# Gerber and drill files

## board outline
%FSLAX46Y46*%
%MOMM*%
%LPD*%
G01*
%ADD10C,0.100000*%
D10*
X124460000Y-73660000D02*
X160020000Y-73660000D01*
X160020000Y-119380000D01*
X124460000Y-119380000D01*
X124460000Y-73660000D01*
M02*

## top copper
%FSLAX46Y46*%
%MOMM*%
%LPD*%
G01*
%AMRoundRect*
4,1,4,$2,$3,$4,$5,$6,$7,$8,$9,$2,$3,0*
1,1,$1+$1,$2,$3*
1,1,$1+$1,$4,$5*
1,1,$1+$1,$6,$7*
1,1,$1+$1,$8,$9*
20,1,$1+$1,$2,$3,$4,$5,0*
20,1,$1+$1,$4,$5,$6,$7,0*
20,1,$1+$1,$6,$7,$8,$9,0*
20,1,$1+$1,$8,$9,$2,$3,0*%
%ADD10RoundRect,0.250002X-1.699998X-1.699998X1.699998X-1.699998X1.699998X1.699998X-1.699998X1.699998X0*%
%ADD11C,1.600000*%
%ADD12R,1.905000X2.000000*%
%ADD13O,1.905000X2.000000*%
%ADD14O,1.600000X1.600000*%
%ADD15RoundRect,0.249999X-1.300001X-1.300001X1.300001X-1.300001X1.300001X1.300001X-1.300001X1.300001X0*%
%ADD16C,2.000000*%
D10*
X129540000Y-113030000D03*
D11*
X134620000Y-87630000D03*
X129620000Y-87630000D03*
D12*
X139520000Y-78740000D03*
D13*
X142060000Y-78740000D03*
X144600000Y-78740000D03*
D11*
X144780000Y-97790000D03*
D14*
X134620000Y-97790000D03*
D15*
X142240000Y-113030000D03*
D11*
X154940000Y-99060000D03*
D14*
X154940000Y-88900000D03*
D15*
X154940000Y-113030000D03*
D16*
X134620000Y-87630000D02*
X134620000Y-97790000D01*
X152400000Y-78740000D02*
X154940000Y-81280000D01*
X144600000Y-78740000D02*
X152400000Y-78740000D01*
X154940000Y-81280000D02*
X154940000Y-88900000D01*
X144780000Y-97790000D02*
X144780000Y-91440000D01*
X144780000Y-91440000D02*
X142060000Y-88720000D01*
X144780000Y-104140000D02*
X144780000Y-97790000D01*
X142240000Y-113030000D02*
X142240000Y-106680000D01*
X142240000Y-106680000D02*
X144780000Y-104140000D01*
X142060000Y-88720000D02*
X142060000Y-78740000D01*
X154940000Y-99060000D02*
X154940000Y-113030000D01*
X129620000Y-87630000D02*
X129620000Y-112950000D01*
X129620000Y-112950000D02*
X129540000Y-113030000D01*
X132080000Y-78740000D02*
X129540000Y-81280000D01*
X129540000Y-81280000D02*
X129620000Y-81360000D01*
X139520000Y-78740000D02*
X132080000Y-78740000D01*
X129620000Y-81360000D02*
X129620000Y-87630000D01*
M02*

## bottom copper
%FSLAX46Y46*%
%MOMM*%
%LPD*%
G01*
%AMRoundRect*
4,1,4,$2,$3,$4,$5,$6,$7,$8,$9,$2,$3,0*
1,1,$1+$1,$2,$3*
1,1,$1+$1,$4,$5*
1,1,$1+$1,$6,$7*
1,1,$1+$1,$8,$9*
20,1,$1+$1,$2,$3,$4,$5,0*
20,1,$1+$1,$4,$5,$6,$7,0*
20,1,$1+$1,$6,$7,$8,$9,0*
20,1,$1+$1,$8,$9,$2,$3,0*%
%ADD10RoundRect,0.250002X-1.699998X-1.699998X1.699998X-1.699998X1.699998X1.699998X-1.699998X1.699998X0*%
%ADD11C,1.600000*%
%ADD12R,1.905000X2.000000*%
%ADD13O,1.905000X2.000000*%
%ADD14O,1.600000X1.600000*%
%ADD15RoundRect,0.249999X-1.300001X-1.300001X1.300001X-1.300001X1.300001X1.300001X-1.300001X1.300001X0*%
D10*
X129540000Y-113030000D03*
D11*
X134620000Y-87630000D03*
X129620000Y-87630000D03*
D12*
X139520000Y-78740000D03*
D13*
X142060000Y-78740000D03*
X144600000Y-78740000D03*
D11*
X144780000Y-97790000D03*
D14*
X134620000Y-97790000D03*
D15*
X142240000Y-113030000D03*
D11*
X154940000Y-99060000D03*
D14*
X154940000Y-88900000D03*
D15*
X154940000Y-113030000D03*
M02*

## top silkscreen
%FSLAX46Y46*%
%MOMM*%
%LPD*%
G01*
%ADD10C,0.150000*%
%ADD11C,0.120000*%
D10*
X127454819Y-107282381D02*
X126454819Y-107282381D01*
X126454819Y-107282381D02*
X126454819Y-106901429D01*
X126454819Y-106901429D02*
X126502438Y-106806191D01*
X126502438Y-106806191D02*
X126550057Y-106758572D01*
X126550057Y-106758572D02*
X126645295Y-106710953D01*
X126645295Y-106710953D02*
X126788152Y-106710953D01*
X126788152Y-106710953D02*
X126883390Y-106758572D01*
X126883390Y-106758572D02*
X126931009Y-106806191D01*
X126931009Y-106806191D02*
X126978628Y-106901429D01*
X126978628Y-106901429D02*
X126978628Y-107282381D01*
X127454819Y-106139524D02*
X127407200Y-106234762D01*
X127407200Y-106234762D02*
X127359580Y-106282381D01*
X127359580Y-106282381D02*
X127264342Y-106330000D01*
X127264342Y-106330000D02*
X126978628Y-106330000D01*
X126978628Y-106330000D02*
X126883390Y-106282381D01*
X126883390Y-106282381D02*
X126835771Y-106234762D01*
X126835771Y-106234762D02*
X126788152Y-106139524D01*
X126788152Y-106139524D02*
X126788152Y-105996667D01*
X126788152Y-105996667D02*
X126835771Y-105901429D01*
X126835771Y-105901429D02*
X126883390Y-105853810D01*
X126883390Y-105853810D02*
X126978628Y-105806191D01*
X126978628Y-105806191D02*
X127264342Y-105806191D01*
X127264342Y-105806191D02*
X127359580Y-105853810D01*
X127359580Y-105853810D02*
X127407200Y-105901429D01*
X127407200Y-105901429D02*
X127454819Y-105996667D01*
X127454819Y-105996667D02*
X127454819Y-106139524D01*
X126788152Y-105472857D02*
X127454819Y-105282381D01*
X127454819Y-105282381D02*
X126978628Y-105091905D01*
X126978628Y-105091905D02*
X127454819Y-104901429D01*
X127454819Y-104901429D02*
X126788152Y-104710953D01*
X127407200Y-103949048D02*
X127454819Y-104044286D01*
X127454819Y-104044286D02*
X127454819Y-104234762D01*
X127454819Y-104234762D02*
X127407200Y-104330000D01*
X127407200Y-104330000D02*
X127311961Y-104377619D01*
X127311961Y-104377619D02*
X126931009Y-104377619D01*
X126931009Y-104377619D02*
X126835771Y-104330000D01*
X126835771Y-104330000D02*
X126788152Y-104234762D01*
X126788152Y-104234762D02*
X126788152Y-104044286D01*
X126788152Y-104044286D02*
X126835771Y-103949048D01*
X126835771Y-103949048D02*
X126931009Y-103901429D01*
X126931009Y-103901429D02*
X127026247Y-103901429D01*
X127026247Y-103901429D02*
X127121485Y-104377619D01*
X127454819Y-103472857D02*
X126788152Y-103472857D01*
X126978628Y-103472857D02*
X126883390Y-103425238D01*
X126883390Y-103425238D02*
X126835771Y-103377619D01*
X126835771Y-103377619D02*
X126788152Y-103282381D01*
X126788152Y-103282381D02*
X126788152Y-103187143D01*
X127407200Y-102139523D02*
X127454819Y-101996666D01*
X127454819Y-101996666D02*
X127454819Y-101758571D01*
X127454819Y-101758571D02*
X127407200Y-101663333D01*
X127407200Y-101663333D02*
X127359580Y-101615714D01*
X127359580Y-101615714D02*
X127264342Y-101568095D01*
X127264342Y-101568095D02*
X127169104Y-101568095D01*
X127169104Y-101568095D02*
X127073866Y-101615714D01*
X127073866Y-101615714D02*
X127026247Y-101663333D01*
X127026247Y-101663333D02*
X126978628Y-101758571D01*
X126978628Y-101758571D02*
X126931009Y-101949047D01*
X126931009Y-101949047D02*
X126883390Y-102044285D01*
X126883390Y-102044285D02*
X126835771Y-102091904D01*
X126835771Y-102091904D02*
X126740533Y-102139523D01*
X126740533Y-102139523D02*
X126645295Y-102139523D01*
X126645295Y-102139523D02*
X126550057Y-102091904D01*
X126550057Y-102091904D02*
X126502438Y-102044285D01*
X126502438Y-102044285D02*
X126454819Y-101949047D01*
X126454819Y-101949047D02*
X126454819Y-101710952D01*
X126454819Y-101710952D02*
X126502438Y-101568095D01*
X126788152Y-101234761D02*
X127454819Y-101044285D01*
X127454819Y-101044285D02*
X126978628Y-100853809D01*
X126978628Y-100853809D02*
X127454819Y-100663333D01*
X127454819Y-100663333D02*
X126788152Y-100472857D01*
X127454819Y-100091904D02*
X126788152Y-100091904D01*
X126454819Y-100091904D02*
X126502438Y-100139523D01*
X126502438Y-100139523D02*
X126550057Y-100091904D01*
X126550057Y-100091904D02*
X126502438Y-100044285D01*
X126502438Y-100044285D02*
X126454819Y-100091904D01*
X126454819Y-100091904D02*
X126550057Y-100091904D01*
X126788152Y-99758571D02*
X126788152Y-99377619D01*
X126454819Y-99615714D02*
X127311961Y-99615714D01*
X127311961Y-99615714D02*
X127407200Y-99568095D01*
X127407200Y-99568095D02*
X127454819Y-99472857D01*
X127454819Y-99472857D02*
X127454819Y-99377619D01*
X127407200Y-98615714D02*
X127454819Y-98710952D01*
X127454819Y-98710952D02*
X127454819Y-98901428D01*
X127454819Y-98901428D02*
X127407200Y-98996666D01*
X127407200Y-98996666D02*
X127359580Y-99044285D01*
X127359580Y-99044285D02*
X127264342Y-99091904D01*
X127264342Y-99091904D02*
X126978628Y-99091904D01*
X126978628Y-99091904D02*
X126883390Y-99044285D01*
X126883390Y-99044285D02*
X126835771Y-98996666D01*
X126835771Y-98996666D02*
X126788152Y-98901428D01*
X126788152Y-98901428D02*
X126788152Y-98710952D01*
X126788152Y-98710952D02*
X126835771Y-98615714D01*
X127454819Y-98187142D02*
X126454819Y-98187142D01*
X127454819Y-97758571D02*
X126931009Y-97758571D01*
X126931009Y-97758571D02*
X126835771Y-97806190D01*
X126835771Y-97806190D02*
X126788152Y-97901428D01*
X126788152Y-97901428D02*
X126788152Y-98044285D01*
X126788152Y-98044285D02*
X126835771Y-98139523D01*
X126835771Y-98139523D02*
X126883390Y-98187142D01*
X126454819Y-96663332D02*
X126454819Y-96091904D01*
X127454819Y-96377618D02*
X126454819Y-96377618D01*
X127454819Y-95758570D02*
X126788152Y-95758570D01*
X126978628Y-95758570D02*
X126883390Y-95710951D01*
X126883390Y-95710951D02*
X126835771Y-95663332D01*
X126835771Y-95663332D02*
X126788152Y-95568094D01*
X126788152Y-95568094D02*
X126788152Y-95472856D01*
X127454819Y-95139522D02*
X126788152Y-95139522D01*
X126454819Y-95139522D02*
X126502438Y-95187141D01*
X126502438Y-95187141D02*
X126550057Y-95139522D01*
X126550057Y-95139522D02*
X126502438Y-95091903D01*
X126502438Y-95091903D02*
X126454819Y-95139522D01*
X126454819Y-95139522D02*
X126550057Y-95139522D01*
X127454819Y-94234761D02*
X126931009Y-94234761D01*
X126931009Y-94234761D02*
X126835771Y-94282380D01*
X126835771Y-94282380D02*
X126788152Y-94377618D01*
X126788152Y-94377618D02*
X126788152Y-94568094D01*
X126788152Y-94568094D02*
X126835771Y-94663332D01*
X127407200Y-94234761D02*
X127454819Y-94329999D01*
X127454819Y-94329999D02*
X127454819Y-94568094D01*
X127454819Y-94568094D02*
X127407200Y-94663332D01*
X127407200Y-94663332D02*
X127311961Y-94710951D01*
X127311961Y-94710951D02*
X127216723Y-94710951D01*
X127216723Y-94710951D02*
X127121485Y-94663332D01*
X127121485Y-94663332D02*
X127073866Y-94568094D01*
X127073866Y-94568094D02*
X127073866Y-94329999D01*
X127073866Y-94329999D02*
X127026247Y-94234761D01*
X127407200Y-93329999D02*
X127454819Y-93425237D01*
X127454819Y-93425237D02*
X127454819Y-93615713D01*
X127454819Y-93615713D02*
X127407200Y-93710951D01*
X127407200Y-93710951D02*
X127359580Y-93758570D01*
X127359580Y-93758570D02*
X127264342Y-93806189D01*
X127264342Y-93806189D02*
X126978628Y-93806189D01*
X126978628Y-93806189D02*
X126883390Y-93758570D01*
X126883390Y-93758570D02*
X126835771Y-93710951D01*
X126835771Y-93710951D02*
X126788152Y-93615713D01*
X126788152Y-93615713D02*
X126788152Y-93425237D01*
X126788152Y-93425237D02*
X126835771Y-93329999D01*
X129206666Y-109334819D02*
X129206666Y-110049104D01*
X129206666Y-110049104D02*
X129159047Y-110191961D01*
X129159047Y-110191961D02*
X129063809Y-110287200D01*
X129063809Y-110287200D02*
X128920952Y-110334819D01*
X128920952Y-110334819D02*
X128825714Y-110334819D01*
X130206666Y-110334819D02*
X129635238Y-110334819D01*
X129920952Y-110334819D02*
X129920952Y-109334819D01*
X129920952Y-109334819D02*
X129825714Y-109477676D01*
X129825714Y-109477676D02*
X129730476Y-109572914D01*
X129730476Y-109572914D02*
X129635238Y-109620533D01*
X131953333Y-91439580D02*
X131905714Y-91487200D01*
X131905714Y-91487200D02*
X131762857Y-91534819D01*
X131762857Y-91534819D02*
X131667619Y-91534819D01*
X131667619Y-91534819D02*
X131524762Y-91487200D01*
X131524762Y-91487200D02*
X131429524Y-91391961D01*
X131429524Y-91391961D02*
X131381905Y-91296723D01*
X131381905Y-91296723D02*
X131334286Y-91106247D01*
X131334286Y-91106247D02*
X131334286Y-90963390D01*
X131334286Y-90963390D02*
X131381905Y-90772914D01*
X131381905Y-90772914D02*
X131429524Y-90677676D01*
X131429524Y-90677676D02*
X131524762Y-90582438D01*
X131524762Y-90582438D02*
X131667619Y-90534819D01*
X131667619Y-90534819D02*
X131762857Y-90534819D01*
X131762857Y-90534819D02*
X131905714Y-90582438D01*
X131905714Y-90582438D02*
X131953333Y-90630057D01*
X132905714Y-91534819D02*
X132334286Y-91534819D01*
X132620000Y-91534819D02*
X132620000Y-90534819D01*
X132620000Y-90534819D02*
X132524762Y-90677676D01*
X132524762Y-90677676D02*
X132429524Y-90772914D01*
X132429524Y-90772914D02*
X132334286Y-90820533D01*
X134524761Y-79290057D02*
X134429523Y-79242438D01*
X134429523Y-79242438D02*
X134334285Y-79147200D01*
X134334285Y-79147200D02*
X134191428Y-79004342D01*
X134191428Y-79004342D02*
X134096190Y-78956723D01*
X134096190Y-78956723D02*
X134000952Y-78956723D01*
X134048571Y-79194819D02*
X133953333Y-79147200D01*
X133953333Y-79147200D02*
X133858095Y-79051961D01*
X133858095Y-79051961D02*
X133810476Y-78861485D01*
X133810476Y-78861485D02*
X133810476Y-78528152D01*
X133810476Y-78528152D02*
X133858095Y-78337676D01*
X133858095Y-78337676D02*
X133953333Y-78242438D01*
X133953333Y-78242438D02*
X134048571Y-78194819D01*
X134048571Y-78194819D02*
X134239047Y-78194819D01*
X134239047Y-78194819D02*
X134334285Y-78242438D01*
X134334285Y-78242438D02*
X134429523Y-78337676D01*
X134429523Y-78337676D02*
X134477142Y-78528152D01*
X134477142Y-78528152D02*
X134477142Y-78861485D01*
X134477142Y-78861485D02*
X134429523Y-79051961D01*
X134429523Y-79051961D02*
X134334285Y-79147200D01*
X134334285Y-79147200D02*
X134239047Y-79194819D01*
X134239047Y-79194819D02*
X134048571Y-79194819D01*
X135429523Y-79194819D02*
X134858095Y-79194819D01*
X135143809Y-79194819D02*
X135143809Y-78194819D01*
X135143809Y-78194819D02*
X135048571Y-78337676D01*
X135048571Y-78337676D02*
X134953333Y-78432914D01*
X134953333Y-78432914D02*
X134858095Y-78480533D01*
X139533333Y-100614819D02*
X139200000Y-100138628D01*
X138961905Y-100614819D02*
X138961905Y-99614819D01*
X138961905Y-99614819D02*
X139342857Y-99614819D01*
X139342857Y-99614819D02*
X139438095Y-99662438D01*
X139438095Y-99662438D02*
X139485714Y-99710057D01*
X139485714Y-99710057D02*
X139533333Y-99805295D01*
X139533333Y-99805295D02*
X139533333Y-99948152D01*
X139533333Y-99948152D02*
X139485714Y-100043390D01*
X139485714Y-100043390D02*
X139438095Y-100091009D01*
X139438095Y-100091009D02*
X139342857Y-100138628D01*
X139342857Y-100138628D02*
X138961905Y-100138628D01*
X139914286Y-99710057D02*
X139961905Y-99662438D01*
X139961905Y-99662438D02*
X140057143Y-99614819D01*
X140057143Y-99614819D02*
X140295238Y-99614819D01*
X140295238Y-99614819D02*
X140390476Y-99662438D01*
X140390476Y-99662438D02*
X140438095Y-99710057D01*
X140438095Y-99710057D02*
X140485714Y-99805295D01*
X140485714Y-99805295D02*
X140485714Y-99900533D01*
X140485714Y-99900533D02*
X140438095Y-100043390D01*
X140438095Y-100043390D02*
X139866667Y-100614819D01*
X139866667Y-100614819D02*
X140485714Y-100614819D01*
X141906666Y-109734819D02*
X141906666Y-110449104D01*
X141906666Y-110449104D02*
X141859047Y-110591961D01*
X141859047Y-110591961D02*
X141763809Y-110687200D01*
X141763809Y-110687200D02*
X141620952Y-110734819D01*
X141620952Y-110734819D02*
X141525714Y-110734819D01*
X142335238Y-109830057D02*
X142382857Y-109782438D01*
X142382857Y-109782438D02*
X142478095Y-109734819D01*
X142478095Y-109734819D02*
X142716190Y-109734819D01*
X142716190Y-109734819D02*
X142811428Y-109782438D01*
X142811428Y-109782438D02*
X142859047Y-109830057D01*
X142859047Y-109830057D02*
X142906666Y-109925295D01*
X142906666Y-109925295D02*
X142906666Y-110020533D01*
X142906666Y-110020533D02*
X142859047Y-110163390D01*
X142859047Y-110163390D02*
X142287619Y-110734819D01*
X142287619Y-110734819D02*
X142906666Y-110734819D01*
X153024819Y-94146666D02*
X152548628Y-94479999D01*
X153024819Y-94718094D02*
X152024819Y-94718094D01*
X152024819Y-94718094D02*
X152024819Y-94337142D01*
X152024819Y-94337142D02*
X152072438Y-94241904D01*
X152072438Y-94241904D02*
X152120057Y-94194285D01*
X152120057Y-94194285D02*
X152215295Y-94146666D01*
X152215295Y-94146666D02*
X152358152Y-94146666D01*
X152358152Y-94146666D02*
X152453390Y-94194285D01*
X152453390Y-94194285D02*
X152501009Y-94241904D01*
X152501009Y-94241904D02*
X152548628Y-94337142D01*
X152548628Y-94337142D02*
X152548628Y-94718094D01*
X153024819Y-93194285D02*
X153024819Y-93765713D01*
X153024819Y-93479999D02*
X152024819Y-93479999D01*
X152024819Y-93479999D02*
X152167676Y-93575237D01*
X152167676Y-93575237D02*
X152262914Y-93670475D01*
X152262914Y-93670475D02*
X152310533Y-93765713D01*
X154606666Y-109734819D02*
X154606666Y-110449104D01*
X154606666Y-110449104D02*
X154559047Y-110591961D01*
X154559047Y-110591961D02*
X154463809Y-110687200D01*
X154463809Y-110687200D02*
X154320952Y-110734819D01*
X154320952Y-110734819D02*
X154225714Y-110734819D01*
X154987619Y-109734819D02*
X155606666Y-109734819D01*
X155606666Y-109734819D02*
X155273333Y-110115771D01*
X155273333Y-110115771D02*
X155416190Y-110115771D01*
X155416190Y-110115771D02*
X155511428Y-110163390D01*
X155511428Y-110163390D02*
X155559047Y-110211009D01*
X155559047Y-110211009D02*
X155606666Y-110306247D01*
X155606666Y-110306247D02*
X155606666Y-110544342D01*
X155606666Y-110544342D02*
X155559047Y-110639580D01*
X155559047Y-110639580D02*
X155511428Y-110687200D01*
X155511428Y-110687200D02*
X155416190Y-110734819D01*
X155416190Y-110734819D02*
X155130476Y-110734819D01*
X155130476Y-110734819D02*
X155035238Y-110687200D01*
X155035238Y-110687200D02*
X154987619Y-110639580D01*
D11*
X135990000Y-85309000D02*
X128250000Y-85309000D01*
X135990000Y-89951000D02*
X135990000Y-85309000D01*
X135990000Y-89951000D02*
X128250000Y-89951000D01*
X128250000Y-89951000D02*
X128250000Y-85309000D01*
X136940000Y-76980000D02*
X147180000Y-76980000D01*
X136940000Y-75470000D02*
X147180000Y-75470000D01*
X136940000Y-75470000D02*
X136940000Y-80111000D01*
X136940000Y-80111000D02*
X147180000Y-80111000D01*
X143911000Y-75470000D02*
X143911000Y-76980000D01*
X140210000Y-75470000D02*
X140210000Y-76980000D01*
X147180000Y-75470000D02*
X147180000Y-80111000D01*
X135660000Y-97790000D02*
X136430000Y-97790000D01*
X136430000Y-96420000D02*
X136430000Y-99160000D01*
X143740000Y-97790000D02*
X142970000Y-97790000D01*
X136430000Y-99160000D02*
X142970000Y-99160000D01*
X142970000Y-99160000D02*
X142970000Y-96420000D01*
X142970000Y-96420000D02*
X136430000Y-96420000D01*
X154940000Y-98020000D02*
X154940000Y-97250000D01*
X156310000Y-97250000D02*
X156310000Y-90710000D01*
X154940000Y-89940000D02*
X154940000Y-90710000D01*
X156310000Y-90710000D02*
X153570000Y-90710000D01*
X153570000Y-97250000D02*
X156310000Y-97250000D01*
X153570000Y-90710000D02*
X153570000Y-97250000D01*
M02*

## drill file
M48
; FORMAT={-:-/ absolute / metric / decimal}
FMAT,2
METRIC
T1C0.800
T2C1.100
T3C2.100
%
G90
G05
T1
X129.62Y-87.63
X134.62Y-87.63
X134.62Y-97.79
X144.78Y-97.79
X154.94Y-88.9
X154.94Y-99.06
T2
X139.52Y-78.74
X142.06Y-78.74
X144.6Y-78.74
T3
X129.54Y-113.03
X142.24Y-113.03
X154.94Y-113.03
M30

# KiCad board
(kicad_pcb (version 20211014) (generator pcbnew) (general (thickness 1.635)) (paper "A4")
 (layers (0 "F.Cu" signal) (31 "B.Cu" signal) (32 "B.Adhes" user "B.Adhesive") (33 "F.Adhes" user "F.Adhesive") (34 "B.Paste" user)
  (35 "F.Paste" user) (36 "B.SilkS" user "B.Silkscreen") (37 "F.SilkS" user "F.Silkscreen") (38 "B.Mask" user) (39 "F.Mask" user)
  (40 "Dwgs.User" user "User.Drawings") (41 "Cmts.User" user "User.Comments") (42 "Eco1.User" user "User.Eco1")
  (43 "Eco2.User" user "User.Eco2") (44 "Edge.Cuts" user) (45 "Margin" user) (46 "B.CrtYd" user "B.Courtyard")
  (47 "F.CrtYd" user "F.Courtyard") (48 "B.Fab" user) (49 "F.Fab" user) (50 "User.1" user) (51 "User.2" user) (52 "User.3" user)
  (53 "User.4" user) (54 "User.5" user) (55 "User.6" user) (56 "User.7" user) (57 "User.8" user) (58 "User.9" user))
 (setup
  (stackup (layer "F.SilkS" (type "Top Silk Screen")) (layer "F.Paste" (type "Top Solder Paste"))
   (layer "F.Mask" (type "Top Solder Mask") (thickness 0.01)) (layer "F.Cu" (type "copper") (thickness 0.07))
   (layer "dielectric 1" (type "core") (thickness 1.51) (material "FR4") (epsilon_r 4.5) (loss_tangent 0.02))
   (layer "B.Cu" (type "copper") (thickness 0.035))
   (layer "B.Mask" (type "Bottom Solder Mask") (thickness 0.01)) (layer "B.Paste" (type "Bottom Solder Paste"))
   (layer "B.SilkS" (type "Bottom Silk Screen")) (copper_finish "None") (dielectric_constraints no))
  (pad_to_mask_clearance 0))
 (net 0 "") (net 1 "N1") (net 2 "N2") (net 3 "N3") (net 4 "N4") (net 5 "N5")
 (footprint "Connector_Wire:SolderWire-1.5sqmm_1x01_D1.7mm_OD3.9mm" (layer "F.Cu") (at 129.54 113.03)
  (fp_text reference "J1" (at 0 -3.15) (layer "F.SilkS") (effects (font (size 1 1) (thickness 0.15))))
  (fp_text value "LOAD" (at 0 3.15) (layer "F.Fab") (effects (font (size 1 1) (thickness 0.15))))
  (pad "1" thru_hole roundrect locked (at 0 0) (size 3.9 3.9) (drill 2.1) (layers *.Cu *.Mask) (roundrect_rratio 0.064103) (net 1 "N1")))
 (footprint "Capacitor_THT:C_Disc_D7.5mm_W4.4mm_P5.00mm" (layer "F.Cu") (at 134.62 87.63 180)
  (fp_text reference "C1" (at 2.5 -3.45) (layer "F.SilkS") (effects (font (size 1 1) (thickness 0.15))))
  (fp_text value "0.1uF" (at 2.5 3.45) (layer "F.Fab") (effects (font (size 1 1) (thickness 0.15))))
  (fp_line (start -1.37 2.321) (end 6.37 2.321) (layer "F.SilkS") (width 0.12))
  (fp_line (start -1.37 -2.321) (end -1.37 2.321) (layer "F.SilkS") (width 0.12))
  (fp_line (start -1.37 -2.321) (end 6.37 -2.321) (layer "F.SilkS") (width 0.12))
  (fp_line (start 6.37 -2.321) (end 6.37 2.321) (layer "F.SilkS") (width 0.12))
  (pad "1" thru_hole circle locked (at 0 0 180) (size 1.6 1.6) (drill 0.8) (layers *.Cu *.Mask) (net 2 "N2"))
  (pad "2" thru_hole circle locked (at 5 0 180) (size 1.6 1.6) (drill 0.8) (layers *.Cu *.Mask) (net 1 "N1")))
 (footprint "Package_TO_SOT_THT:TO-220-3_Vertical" (layer "F.Cu") (at 139.52 78.74)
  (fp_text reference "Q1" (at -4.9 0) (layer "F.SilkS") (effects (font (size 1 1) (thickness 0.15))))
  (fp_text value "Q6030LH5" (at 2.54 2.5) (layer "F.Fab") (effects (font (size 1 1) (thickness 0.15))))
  (fp_line (start -2.58 -1.76) (end 7.66 -1.76) (layer "F.SilkS") (width 0.12))
  (fp_line (start -2.58 -3.27) (end 7.66 -3.27) (layer "F.SilkS") (width 0.12))
  (fp_line (start -2.58 -3.27) (end -2.58 1.371) (layer "F.SilkS") (width 0.12))
  (fp_line (start -2.58 1.371) (end 7.66 1.371) (layer "F.SilkS") (width 0.12))
  (fp_line (start 4.391 -3.27) (end 4.391 -1.76) (layer "F.SilkS") (width 0.12))
  (fp_line (start 0.69 -3.27) (end 0.69 -1.76) (layer "F.SilkS") (width 0.12))
  (fp_line (start 7.66 -3.27) (end 7.66 1.371) (layer "F.SilkS") (width 0.12))
  (pad "1" thru_hole rect locked (at 0 0) (size 1.905 2) (drill 1.1) (layers *.Cu *.Mask) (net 1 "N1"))
  (pad "2" thru_hole oval locked (at 2.54 0) (size 1.905 2) (drill 1.1) (layers *.Cu *.Mask) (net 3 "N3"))
  (pad "3" thru_hole oval locked (at 5.08 0) (size 1.905 2) (drill 1.1) (layers *.Cu *.Mask) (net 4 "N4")))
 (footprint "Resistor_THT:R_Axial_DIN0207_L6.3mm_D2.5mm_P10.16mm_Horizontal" (layer "F.Cu") (at 144.78 97.79 180)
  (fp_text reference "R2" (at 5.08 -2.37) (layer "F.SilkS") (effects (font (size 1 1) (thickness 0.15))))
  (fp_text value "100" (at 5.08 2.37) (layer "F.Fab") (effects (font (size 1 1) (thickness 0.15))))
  (fp_line (start 9.12 0) (end 8.35 0) (layer "F.SilkS") (width 0.12))
  (fp_line (start 8.35 1.37) (end 8.35 -1.37) (layer "F.SilkS") (width 0.12))
  (fp_line (start 1.04 0) (end 1.81 0) (layer "F.SilkS") (width 0.12))
  (fp_line (start 8.35 -1.37) (end 1.81 -1.37) (layer "F.SilkS") (width 0.12))
  (fp_line (start 1.81 -1.37) (end 1.81 1.37) (layer "F.SilkS") (width 0.12))
  (fp_line (start 1.81 1.37) (end 8.35 1.37) (layer "F.SilkS") (width 0.12))
  (pad "1" thru_hole circle locked (at 0 0 180) (size 1.6 1.6) (drill 0.8) (layers *.Cu *.Mask) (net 3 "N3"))
  (pad "2" thru_hole oval locked (at 10.16 0 180) (size 1.6 1.6) (drill 0.8) (layers *.Cu *.Mask) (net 2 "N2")))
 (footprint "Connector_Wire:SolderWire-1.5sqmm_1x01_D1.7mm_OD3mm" (layer "F.Cu") (at 142.24 113.03)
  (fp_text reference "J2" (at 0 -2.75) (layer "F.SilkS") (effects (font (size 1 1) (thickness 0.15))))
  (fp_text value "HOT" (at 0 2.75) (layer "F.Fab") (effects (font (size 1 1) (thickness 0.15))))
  (pad "1" thru_hole roundrect locked (at 0 0) (size 3.1 3.1) (drill 2.1) (layers *.Cu *.Mask) (roundrect_rratio 0.080645) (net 3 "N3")))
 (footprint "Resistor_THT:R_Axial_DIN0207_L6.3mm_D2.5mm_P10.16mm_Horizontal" (layer "F.Cu") (at 154.94 99.06 90)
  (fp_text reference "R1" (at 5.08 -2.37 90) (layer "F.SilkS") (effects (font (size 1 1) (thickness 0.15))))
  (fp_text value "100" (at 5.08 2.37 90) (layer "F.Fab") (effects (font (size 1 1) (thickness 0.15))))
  (fp_line (start 1.04 0) (end 1.81 0) (layer "F.SilkS") (width 0.12))
  (fp_line (start 1.81 1.37) (end 8.35 1.37) (layer "F.SilkS") (width 0.12))
  (fp_line (start 9.12 0) (end 8.35 0) (layer "F.SilkS") (width 0.12))
  (fp_line (start 8.35 1.37) (end 8.35 -1.37) (layer "F.SilkS") (width 0.12))
  (fp_line (start 1.81 -1.37) (end 1.81 1.37) (layer "F.SilkS") (width 0.12))
  (fp_line (start 8.35 -1.37) (end 1.81 -1.37) (layer "F.SilkS") (width 0.12))
  (pad "1" thru_hole circle locked (at 0 0 90) (size 1.6 1.6) (drill 0.8) (layers *.Cu *.Mask) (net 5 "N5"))
  (pad "2" thru_hole oval locked (at 10.16 0 90) (size 1.6 1.6) (drill 0.8) (layers *.Cu *.Mask) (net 4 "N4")))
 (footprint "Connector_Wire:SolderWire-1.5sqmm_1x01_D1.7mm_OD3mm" (layer "F.Cu") (at 154.94 113.03)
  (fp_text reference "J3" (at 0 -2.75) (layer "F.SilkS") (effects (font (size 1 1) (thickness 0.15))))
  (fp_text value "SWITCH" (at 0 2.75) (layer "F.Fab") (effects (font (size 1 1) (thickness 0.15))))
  (pad "1" thru_hole roundrect locked (at 0 0) (size 3.1 3.1) (drill 2.1) (layers *.Cu *.Mask) (roundrect_rratio 0.080645) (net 5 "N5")))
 (gr_rect (start 124.46 73.66) (end 160.02 119.38) (layer "Edge.Cuts") (width 0.1) (fill none))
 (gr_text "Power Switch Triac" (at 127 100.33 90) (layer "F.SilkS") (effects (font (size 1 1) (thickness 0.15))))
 (segment (start 134.62 87.63) (end 134.62 97.79) (width 2) (layer "F.Cu") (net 2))
 (segment (start 152.4 78.74) (end 154.94 81.28) (width 2) (layer "F.Cu") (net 4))
 (segment (start 144.6 78.74) (end 152.4 78.74) (width 2) (layer "F.Cu") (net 4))
 (segment (start 154.94 81.28) (end 154.94 88.9) (width 2) (layer "F.Cu") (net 4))
 (segment (start 144.78 97.79) (end 144.78 91.44) (width 2) (layer "F.Cu") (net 3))
 (segment (start 144.78 91.44) (end 142.06 88.72) (width 2) (layer "F.Cu") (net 3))
 (segment (start 144.78 104.14) (end 144.78 97.79) (width 2) (layer "F.Cu") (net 3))
 (segment (start 142.24 113.03) (end 142.24 106.68) (width 2) (layer "F.Cu") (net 3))
 (segment (start 142.24 106.68) (end 144.78 104.14) (width 2) (layer "F.Cu") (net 3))
 (segment (start 142.06 88.72) (end 142.06 78.74) (width 2) (layer "F.Cu") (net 3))
 (segment (start 154.94 99.06) (end 154.94 113.03) (width 2) (layer "F.Cu") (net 5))
 (segment (start 129.62 87.63) (end 129.62 112.95) (width 2) (layer "F.Cu") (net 1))
 (segment (start 129.62 112.95) (end 129.54 113.03) (width 2) (layer "F.Cu") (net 1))
 (segment (start 132.08 78.74) (end 129.54 81.28) (width 2) (layer "F.Cu") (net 1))
 (segment (start 129.54 81.28) (end 129.62 81.36) (width 2) (layer "F.Cu") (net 1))
 (segment (start 139.52 78.74) (end 132.08 78.74) (width 2) (layer "F.Cu") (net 1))
 (segment (start 129.62 81.36) (end 129.62 87.63) (width 2) (layer "F.Cu") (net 1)))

